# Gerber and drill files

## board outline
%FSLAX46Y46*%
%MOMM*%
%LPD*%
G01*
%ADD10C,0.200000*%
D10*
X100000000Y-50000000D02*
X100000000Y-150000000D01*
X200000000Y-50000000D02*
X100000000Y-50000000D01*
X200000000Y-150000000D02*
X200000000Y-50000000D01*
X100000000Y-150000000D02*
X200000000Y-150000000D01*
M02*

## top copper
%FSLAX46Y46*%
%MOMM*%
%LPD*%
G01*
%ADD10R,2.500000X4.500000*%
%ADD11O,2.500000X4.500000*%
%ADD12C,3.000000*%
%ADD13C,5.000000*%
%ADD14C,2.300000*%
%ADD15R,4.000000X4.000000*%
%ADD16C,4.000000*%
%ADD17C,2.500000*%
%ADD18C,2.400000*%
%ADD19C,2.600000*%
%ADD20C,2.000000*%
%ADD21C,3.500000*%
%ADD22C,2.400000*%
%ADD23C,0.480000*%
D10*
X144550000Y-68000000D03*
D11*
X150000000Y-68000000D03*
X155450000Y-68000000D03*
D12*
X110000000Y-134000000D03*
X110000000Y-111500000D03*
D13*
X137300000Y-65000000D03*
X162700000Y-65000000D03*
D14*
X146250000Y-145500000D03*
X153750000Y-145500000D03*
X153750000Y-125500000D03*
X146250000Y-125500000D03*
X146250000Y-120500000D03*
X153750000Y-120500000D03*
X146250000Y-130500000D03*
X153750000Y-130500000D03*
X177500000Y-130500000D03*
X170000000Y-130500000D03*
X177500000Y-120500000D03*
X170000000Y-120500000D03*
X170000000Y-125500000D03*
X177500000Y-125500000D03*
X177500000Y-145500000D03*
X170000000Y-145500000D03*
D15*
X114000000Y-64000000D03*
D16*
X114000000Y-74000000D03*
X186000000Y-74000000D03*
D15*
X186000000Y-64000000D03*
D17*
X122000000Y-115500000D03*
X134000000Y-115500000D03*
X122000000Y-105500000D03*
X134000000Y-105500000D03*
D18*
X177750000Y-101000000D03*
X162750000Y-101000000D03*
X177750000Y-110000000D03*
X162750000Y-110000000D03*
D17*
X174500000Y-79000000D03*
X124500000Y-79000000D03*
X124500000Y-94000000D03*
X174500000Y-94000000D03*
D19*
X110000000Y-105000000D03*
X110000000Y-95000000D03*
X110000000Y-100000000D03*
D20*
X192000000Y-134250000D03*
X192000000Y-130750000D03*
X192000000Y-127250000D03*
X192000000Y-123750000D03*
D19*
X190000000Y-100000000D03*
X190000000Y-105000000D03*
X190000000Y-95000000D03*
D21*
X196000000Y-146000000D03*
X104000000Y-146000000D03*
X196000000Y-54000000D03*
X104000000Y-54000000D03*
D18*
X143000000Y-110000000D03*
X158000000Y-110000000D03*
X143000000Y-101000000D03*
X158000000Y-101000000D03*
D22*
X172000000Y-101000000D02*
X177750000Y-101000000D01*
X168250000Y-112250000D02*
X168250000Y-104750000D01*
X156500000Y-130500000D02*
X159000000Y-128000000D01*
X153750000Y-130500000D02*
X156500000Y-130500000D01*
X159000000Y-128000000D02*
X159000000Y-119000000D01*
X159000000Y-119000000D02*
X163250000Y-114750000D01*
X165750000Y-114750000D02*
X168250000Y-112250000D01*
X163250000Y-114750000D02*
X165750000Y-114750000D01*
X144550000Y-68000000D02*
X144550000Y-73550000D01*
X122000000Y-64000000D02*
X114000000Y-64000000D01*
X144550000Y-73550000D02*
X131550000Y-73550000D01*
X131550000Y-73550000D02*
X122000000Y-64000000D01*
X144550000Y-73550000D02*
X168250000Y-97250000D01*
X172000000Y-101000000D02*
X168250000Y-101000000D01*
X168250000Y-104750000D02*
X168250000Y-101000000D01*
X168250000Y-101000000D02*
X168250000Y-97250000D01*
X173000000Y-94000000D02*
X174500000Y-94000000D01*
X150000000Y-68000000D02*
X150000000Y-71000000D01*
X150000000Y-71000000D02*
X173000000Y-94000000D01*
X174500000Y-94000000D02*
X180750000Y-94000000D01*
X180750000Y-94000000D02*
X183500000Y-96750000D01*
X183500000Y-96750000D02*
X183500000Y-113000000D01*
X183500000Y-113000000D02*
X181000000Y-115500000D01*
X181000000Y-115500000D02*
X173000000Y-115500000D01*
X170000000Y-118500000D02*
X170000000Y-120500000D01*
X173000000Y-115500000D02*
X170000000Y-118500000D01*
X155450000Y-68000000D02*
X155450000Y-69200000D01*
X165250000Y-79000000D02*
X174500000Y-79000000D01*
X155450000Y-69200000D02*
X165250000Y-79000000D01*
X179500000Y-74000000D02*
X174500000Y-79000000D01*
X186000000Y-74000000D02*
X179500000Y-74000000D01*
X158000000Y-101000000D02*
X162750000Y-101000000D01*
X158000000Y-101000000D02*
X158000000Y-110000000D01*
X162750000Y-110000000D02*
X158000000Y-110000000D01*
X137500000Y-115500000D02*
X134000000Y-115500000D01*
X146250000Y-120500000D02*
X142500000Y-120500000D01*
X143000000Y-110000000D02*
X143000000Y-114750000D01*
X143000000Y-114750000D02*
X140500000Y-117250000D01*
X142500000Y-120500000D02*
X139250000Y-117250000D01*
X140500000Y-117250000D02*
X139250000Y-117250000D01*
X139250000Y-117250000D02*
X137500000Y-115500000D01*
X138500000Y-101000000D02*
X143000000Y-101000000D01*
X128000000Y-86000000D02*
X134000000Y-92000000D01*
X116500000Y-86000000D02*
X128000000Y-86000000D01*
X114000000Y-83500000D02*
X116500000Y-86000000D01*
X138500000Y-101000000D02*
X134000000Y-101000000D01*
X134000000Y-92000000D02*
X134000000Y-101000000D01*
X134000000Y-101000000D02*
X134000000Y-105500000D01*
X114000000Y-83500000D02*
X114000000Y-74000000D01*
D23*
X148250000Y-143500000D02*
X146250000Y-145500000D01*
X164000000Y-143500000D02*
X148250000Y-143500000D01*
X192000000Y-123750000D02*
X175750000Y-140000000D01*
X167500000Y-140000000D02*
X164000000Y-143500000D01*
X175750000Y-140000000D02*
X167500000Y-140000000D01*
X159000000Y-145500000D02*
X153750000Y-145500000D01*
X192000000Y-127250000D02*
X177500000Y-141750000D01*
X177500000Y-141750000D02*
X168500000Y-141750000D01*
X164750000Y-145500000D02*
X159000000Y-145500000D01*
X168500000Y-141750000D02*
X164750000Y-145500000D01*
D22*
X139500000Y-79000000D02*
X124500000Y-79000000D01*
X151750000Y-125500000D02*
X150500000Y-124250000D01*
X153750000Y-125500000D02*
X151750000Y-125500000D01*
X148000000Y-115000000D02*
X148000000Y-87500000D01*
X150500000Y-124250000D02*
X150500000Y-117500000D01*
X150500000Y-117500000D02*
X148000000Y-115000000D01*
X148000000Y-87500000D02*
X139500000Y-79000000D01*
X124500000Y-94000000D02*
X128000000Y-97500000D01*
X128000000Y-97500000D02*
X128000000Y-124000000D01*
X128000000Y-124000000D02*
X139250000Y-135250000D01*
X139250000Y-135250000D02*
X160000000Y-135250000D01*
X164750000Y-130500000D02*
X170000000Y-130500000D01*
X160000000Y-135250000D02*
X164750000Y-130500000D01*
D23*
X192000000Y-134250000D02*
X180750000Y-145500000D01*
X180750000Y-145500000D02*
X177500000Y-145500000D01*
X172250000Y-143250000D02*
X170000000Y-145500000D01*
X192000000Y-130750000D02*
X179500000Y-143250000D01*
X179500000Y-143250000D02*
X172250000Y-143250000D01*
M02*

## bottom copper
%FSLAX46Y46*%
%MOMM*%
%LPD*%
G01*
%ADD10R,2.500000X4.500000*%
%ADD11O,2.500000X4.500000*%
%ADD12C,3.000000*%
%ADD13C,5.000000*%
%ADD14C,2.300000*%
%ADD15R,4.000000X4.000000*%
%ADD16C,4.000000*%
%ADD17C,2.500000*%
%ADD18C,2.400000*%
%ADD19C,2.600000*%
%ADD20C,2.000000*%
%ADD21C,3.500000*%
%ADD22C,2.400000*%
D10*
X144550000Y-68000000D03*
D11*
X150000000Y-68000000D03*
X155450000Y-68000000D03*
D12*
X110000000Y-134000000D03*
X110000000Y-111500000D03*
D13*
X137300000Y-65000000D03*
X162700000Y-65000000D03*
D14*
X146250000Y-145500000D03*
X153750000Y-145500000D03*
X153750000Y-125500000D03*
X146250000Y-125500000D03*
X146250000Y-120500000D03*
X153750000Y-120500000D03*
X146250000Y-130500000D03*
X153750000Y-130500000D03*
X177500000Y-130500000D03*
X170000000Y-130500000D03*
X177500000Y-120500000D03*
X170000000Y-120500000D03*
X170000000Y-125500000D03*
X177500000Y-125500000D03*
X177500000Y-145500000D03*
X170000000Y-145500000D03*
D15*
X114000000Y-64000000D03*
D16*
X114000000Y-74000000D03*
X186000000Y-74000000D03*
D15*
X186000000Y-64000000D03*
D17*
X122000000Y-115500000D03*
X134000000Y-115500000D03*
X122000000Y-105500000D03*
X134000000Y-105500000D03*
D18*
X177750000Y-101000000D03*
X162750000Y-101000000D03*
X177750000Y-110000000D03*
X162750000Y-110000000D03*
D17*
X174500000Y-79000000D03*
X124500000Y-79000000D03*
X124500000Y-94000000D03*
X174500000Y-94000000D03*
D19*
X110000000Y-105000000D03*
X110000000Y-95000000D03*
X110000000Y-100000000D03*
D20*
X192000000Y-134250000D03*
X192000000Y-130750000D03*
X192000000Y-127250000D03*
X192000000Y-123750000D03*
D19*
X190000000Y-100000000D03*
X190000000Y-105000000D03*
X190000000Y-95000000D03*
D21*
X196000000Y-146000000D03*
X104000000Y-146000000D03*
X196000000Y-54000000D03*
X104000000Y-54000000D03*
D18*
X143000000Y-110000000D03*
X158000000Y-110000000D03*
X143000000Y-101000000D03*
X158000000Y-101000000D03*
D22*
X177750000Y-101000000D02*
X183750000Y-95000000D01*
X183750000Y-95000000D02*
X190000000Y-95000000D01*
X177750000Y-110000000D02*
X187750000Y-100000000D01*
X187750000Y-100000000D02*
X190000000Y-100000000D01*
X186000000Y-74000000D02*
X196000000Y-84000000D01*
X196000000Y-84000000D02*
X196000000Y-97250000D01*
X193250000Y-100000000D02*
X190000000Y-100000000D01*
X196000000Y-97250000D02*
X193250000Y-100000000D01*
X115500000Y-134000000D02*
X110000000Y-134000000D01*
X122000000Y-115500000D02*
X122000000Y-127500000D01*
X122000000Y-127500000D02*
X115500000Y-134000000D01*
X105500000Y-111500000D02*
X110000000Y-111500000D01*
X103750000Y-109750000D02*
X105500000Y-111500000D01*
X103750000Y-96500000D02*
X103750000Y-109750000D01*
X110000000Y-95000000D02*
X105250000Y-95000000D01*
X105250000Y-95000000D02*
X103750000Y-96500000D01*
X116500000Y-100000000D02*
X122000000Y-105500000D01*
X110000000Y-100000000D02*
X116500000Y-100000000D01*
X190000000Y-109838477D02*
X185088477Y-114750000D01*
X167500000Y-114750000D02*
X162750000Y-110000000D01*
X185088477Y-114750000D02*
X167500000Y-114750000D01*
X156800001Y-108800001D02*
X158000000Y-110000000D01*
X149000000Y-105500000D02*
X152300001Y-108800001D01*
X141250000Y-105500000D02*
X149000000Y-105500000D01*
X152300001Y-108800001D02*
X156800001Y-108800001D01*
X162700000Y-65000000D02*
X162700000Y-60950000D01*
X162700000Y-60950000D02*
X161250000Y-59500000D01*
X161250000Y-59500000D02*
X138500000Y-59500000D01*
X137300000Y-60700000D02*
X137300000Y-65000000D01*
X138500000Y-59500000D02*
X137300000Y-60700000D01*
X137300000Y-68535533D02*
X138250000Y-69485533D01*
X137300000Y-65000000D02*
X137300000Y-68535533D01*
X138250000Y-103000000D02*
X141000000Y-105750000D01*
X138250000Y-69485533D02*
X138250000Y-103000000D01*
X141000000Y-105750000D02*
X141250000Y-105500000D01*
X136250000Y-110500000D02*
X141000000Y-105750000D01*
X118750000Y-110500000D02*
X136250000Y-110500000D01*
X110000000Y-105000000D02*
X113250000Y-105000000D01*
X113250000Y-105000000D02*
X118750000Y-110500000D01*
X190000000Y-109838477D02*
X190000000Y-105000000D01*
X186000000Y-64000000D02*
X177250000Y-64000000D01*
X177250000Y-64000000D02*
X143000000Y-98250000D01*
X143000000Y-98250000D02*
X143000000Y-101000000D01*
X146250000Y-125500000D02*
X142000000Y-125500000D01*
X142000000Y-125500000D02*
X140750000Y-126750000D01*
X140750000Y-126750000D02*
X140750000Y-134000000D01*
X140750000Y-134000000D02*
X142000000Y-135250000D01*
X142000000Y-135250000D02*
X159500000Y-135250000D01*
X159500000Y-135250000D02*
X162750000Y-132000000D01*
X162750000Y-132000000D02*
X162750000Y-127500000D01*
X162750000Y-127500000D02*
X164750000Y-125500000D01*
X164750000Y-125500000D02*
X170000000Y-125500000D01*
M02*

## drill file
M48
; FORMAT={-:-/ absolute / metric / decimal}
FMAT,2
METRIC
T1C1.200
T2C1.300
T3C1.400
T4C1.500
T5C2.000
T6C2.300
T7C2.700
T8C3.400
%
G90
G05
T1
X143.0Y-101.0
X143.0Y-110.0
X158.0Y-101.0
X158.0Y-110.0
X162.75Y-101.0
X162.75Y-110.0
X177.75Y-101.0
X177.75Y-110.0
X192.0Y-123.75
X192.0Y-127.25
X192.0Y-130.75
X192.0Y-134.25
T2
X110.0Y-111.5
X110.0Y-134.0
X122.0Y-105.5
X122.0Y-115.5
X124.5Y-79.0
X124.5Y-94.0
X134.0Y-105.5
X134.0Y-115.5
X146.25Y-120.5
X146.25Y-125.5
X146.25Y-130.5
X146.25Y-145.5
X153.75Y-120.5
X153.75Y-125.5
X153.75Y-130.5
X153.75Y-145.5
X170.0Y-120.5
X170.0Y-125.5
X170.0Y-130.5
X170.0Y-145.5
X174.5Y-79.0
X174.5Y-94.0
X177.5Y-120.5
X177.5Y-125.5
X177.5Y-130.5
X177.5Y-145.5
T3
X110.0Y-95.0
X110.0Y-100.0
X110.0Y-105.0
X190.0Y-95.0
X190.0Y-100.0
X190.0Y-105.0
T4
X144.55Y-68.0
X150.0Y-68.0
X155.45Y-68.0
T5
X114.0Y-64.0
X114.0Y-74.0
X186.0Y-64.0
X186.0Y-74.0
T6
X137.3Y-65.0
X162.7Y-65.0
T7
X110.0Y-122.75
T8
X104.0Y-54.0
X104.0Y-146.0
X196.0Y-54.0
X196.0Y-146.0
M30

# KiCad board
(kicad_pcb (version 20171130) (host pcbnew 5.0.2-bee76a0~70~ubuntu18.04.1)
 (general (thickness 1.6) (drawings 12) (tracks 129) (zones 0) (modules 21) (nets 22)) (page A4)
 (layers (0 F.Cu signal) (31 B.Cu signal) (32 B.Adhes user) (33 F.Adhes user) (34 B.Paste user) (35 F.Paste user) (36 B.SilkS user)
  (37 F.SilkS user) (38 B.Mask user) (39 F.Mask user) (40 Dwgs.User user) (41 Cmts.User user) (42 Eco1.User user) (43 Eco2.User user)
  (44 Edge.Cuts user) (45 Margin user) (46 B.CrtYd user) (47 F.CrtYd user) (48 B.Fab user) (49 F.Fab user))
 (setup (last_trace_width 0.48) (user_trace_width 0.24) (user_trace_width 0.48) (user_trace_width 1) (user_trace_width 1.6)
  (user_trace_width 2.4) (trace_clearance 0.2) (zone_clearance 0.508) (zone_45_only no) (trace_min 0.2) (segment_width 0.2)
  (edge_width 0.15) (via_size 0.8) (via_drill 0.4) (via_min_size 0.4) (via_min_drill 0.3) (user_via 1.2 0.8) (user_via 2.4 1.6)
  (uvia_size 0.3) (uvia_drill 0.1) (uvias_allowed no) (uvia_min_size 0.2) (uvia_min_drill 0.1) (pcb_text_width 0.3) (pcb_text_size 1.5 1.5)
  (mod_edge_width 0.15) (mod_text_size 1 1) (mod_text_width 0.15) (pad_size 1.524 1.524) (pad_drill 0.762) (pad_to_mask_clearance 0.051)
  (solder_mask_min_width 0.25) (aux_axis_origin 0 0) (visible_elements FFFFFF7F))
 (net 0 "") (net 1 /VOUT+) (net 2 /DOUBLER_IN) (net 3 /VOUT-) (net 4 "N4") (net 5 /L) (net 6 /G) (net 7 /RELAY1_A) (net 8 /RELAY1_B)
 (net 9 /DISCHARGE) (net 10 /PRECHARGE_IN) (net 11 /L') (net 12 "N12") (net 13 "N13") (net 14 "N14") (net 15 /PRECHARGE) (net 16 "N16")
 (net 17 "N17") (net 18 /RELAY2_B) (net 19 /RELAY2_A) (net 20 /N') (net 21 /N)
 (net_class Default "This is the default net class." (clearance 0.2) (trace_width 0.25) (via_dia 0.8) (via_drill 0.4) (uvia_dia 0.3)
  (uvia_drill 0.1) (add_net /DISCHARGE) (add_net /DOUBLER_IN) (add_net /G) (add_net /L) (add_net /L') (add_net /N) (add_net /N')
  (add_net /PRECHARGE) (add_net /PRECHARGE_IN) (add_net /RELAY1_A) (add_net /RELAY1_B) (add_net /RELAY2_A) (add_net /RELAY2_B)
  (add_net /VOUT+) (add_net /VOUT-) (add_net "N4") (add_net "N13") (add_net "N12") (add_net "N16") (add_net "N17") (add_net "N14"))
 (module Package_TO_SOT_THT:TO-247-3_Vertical (layer F.Cu) (at 144.55 68)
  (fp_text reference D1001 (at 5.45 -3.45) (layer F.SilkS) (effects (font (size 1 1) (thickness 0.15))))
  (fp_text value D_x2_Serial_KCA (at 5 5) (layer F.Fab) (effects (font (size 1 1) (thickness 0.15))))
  (pad 1 thru_hole rect (at 0 0) (size 2.5 4.5) (drill 1.5) (layers *.Cu *.Mask) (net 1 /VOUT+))
  (pad 2 thru_hole oval (at 5.45 0) (size 2.5 4.5) (drill 1.5) (layers *.Cu *.Mask) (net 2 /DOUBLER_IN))
  (pad 3 thru_hole oval (at 10.9 0) (size 2.5 4.5) (drill 1.5) (layers *.Cu *.Mask) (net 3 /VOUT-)))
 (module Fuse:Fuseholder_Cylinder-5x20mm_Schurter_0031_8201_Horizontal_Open (layer F.Cu) (at 110 134 90)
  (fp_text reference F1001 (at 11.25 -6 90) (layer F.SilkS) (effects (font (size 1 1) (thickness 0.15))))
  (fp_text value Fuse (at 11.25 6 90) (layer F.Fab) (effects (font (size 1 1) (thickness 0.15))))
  (pad 1 thru_hole circle (at 0 0 90) (size 3 3) (drill 1.3) (layers *.Cu *.Mask) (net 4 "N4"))
  (pad 2 thru_hole circle (at 22.5 0 90) (size 3 3) (drill 1.3) (layers *.Cu *.Mask) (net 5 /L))
  (pad "" np_thru_hole circle (at 11.25 0 90) (size 2.7 2.7) (drill 2.7) (layers *.Cu *.Mask)))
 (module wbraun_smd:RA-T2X (layer F.Cu) (at 150 68)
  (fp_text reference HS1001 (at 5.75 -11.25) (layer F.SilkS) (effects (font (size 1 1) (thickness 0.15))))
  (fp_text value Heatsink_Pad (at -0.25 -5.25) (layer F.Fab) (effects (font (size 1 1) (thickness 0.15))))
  (pad 1 thru_hole circle (at -12.7 -3) (size 5 5) (drill 2.3) (layers *.Cu *.Mask) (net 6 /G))
  (pad 1 thru_hole circle (at 12.7 -3) (size 5 5) (drill 2.3) (layers *.Cu *.Mask) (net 6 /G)))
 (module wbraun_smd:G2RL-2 (layer F.Cu) (at 150 133 90)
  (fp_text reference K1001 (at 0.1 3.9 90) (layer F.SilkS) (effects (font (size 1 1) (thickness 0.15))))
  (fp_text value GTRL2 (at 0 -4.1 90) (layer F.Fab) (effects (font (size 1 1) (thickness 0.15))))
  (pad 1 thru_hole circle (at -12.5 -3.75 90) (size 2.3 2.3) (drill 1.3) (layers *.Cu *.Mask) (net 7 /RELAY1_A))
  (pad 8 thru_hole circle (at -12.5 3.75 90) (size 2.3 2.3) (drill 1.3) (layers *.Cu *.Mask) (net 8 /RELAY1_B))
  (pad 6 thru_hole circle (at 7.5 3.75 90) (size 2.3 2.3) (drill 1.3) (layers *.Cu *.Mask) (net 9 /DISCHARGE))
  (pad 3 thru_hole circle (at 7.5 -3.75 90) (size 2.3 2.3) (drill 1.3) (layers *.Cu *.Mask) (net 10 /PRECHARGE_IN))
  (pad 4 thru_hole circle (at 12.5 -3.75 90) (size 2.3 2.3) (drill 1.3) (layers *.Cu *.Mask) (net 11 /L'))
  (pad 5 thru_hole circle (at 12.5 3.75 90) (size 2.3 2.3) (drill 1.3) (layers *.Cu *.Mask) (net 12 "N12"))
  (pad 2 thru_hole circle (at 2.5 -3.75 90) (size 2.3 2.3) (drill 1.3) (layers *.Cu *.Mask) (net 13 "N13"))
  (pad 7 thru_hole circle (at 2.5 3.75 90) (size 2.3 2.3) (drill 1.3) (layers *.Cu *.Mask) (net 1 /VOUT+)))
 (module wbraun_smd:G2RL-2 (layer F.Cu) (at 173.75 133 90)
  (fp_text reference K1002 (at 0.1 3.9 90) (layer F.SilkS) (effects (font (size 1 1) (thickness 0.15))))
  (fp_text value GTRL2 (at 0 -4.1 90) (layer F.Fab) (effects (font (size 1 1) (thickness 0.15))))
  (pad 7 thru_hole circle (at 2.5 3.75 90) (size 2.3 2.3) (drill 1.3) (layers *.Cu *.Mask) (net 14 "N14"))
  (pad 2 thru_hole circle (at 2.5 -3.75 90) (size 2.3 2.3) (drill 1.3) (layers *.Cu *.Mask) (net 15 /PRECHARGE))
  (pad 5 thru_hole circle (at 12.5 3.75 90) (size 2.3 2.3) (drill 1.3) (layers *.Cu *.Mask) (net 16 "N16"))
  (pad 4 thru_hole circle (at 12.5 -3.75 90) (size 2.3 2.3) (drill 1.3) (layers *.Cu *.Mask) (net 2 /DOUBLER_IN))
  (pad 3 thru_hole circle (at 7.5 -3.75 90) (size 2.3 2.3) (drill 1.3) (layers *.Cu *.Mask) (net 10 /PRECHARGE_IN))
  (pad 6 thru_hole circle (at 7.5 3.75 90) (size 2.3 2.3) (drill 1.3) (layers *.Cu *.Mask) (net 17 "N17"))
  (pad 8 thru_hole circle (at -12.5 3.75 90) (size 2.3 2.3) (drill 1.3) (layers *.Cu *.Mask) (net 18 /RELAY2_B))
  (pad 1 thru_hole circle (at -12.5 -3.75 90) (size 2.3 2.3) (drill 1.3) (layers *.Cu *.Mask) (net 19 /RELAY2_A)))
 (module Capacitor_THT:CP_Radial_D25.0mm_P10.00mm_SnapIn (layer F.Cu) (at 114 64 270)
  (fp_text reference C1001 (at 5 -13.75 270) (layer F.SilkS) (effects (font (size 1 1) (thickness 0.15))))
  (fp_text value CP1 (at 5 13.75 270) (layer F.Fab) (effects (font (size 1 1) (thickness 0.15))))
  (pad 1 thru_hole rect (at 0 0 270) (size 4 4) (drill 2) (layers *.Cu *.Mask) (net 1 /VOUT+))
  (pad 2 thru_hole circle (at 10 0 270) (size 4 4) (drill 2) (layers *.Cu *.Mask) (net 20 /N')))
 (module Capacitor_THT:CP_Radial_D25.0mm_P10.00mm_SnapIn (layer F.Cu) (at 186 64 270)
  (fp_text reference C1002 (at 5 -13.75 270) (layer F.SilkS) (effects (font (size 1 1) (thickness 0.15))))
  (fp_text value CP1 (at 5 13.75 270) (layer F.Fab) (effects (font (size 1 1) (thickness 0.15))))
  (pad 2 thru_hole circle (at 10 0 270) (size 4 4) (drill 2) (layers *.Cu *.Mask) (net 3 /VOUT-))
  (pad 1 thru_hole rect (at 0 0 270) (size 4 4) (drill 2) (layers *.Cu *.Mask) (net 20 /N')))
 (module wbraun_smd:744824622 (layer F.Cu) (at 128 110.5 90)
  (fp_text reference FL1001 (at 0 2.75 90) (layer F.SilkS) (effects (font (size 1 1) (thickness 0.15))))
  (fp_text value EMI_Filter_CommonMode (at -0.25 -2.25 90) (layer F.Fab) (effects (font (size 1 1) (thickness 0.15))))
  (pad 1 thru_hole circle (at -5 -6 90) (size 2.5 2.5) (drill 1.3) (layers *.Cu *.Mask) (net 4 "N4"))
  (pad 2 thru_hole circle (at -5 6 90) (size 2.5 2.5) (drill 1.3) (layers *.Cu *.Mask) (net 11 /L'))
  (pad 3 thru_hole circle (at 5 -6 90) (size 2.5 2.5) (drill 1.3) (layers *.Cu *.Mask) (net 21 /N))
  (pad 4 thru_hole circle (at 5 6 90) (size 2.5 2.5) (drill 1.3) (layers *.Cu *.Mask) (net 20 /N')))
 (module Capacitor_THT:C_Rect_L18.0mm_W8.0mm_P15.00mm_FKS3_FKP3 (layer F.Cu) (at 177.75 101 180)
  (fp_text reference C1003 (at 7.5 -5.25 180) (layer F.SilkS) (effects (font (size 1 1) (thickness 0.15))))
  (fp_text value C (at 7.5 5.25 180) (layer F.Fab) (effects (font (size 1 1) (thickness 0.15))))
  (pad 1 thru_hole circle (at 0 0 180) (size 2.4 2.4) (drill 1.2) (layers *.Cu *.Mask) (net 1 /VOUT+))
  (pad 2 thru_hole circle (at 15 0 180) (size 2.4 2.4) (drill 1.2) (layers *.Cu *.Mask) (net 6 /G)))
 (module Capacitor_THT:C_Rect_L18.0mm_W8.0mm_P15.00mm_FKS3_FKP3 (layer F.Cu) (at 162.75 110)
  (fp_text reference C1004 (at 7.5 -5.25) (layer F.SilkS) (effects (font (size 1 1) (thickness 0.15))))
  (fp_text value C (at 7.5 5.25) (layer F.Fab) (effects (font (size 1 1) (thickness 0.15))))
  (pad 2 thru_hole circle (at 15 0) (size 2.4 2.4) (drill 1.2) (layers *.Cu *.Mask) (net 3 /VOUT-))
  (pad 1 thru_hole circle (at 0 0) (size 2.4 2.4) (drill 1.2) (layers *.Cu *.Mask) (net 6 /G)))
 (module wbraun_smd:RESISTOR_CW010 (layer B.Cu) (at 149.5 79 180)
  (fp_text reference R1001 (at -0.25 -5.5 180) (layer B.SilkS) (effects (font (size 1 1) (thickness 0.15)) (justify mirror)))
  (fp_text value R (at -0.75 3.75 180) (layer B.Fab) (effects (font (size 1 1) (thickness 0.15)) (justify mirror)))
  (pad 1 thru_hole circle (at -25 0 180) (size 2.5 2.5) (drill 1.3) (layers *.Cu *.Mask) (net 3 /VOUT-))
  (pad 2 thru_hole circle (at 25 0 180) (size 2.5 2.5) (drill 1.3) (layers *.Cu *.Mask) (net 9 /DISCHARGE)))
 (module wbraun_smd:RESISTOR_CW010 (layer B.Cu) (at 149.5 94 180)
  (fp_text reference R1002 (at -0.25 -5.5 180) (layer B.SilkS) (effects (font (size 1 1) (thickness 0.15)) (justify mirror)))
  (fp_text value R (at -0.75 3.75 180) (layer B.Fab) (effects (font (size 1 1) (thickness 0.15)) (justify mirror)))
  (pad 2 thru_hole circle (at 25 0 180) (size 2.5 2.5) (drill 1.3) (layers *.Cu *.Mask) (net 15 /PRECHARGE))
  (pad 1 thru_hole circle (at -25 0 180) (size 2.5 2.5) (drill 1.3) (layers *.Cu *.Mask) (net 2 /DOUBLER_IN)))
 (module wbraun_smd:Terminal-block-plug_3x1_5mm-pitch (layer F.Cu) (at 110 100 90)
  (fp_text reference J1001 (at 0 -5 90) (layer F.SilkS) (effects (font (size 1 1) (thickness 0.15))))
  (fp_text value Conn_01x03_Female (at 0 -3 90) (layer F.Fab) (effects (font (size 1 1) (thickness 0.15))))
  (pad 1 thru_hole circle (at -5 0 90) (size 2.6 2.6) (drill 1.4) (layers *.Cu *.Mask) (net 6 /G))
  (pad 3 thru_hole circle (at 5 0 90) (size 2.6 2.6) (drill 1.4) (layers *.Cu *.Mask) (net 5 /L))
  (pad 2 thru_hole circle (at 0 0 90) (size 2.6 2.6) (drill 1.4) (layers *.Cu *.Mask) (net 21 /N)))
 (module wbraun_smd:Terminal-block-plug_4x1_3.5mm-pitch (layer F.Cu) (at 192 129 270)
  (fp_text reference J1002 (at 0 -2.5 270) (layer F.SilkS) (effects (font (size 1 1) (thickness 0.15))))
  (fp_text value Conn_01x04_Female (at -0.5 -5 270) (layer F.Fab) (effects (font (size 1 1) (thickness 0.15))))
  (pad 4 thru_hole circle (at 5.25 0 270) (size 2 2) (drill 1.2) (layers *.Cu *.Mask) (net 18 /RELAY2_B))
  (pad 3 thru_hole circle (at 1.75 0 270) (size 2 2) (drill 1.2) (layers *.Cu *.Mask) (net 19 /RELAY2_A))
  (pad 2 thru_hole circle (at -1.75 0 270) (size 2 2) (drill 1.2) (layers *.Cu *.Mask) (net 8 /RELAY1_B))
  (pad 1 thru_hole circle (at -5.25 0 270) (size 2 2) (drill 1.2) (layers *.Cu *.Mask) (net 7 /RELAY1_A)))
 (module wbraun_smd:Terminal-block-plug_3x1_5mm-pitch (layer F.Cu) (at 190 100 270)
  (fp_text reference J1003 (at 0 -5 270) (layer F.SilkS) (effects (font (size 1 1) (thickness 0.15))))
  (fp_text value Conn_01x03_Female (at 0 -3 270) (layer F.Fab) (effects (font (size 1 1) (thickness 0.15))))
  (pad 2 thru_hole circle (at 0 0 270) (size 2.6 2.6) (drill 1.4) (layers *.Cu *.Mask) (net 3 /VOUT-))
  (pad 3 thru_hole circle (at 5 0 270) (size 2.6 2.6) (drill 1.4) (layers *.Cu *.Mask) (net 6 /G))
  (pad 1 thru_hole circle (at -5 0 270) (size 2.6 2.6) (drill 1.4) (layers *.Cu *.Mask) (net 1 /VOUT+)))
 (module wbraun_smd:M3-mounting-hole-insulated (layer F.Cu) (at 196 146)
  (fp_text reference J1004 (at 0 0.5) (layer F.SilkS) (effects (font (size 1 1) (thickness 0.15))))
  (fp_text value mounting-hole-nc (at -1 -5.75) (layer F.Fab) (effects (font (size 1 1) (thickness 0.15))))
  (pad "" np_thru_hole circle (at 0 0) (size 3.5 3.5) (drill 3.4) (layers *.Cu *.Mask)))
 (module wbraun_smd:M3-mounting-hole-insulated (layer F.Cu) (at 104 146)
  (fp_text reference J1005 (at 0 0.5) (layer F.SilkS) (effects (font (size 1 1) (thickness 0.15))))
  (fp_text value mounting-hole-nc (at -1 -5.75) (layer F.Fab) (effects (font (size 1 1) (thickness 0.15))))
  (pad "" np_thru_hole circle (at 0 0) (size 3.5 3.5) (drill 3.4) (layers *.Cu *.Mask)))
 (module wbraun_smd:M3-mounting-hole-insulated (layer F.Cu) (at 196 54)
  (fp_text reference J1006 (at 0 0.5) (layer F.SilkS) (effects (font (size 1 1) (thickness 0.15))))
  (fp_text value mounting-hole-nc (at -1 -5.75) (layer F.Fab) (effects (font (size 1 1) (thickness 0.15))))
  (pad "" np_thru_hole circle (at 0 0) (size 3.5 3.5) (drill 3.4) (layers *.Cu *.Mask)))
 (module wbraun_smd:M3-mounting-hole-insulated (layer F.Cu) (at 104 54)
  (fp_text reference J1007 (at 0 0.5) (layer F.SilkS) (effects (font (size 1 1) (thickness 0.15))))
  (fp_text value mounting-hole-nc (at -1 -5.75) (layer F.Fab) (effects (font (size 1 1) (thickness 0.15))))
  (pad "" np_thru_hole circle (at 0 0) (size 3.5 3.5) (drill 3.4) (layers *.Cu *.Mask)))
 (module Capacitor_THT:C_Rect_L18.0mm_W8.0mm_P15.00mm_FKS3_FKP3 (layer F.Cu) (at 143 110)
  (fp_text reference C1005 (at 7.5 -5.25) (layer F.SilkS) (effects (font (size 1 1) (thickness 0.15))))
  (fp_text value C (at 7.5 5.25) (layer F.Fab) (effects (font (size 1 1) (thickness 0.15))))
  (pad 1 thru_hole circle (at 0 0) (size 2.4 2.4) (drill 1.2) (layers *.Cu *.Mask) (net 11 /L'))
  (pad 2 thru_hole circle (at 15 0) (size 2.4 2.4) (drill 1.2) (layers *.Cu *.Mask) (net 6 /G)))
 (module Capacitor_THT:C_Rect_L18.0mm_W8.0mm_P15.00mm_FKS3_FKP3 (layer F.Cu) (at 158 101 180)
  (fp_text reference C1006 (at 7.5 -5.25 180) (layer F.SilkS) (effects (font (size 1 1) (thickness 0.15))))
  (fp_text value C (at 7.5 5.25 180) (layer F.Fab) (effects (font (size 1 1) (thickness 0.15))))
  (pad 2 thru_hole circle (at 15 0 180) (size 2.4 2.4) (drill 1.2) (layers *.Cu *.Mask) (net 20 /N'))
  (pad 1 thru_hole circle (at 0 0 180) (size 2.4 2.4) (drill 1.2) (layers *.Cu *.Mask) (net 6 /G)))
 (gr_line (start 100 50) (end 100 150) (layer Edge.Cuts) (width 0.2))
 (gr_line (start 200 50) (end 100 50) (layer Edge.Cuts) (width 0.2))
 (gr_line (start 200 150) (end 200 50) (layer Edge.Cuts) (width 0.2))
 (gr_line (start 100 150) (end 200 150) (layer Edge.Cuts) (width 0.2))
 (segment (start 172 101) (end 177.75 101) (width 2.4) (layer F.Cu) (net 1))
 (segment (start 168.25 112.25) (end 168.25 104.75) (width 2.4) (layer F.Cu) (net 1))
 (segment (start 156.5 130.5) (end 159 128) (width 2.4) (layer F.Cu) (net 1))
 (segment (start 153.75 130.5) (end 156.5 130.5) (width 2.4) (layer F.Cu) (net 1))
 (segment (start 159 128) (end 159 119) (width 2.4) (layer F.Cu) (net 1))
 (segment (start 159 119) (end 163.25 114.75) (width 2.4) (layer F.Cu) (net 1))
 (segment (start 165.75 114.75) (end 168.25 112.25) (width 2.4) (layer F.Cu) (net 1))
 (segment (start 163.25 114.75) (end 165.75 114.75) (width 2.4) (layer F.Cu) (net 1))
 (segment (start 144.55 68) (end 144.55 73.55) (width 2.4) (layer F.Cu) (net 1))
 (segment (start 122 64) (end 114 64) (width 2.4) (layer F.Cu) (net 1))
 (segment (start 144.55 73.55) (end 131.55 73.55) (width 2.4) (layer F.Cu) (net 1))
 (segment (start 131.55 73.55) (end 122 64) (width 2.4) (layer F.Cu) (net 1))
 (segment (start 177.75 101) (end 183.75 95) (width 2.4) (layer B.Cu) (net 1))
 (segment (start 183.75 95) (end 190 95) (width 2.4) (layer B.Cu) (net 1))
 (segment (start 144.55 73.55) (end 168.25 97.25) (width 2.4) (layer F.Cu) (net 1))
 (segment (start 172 101) (end 168.25 101) (width 2.4) (layer F.Cu) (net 1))
 (segment (start 168.25 104.75) (end 168.25 101) (width 2.4) (layer F.Cu) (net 1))
 (segment (start 168.25 101) (end 168.25 97.25) (width 2.4) (layer F.Cu) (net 1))
 (segment (start 173 94) (end 174.5 94) (width 2.4) (layer F.Cu) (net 2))
 (segment (start 150 68) (end 150 71) (width 2.4) (layer F.Cu) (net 2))
 (segment (start 150 71) (end 173 94) (width 2.4) (layer F.Cu) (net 2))
 (segment (start 174.5 94) (end 180.75 94) (width 2.4) (layer F.Cu) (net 2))
 (segment (start 180.75 94) (end 183.5 96.75) (width 2.4) (layer F.Cu) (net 2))
 (segment (start 183.5 96.75) (end 183.5 113) (width 2.4) (layer F.Cu) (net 2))
 (segment (start 183.5 113) (end 181 115.5) (width 2.4) (layer F.Cu) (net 2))
 (segment (start 181 115.5) (end 173 115.5) (width 2.4) (layer F.Cu) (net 2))
 (segment (start 170 118.5) (end 170 120.5) (width 2.4) (layer F.Cu) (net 2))
 (segment (start 173 115.5) (end 170 118.5) (width 2.4) (layer F.Cu) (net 2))
 (segment (start 155.45 68) (end 155.45 69.2) (width 2.4) (layer F.Cu) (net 3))
 (segment (start 165.25 79) (end 174.5 79) (width 2.4) (layer F.Cu) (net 3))
 (segment (start 155.45 69.2) (end 165.25 79) (width 2.4) (layer F.Cu) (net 3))
 (segment (start 179.5 74) (end 174.5 79) (width 2.4) (layer F.Cu) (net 3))
 (segment (start 186 74) (end 179.5 74) (width 2.4) (layer F.Cu) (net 3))
 (segment (start 177.75 110) (end 187.75 100) (width 2.4) (layer B.Cu) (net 3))
 (segment (start 187.75 100) (end 190 100) (width 2.4) (layer B.Cu) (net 3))
 (segment (start 186 74) (end 196 84) (width 2.4) (layer B.Cu) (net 3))
 (segment (start 196 84) (end 196 97.25) (width 2.4) (layer B.Cu) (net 3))
 (segment (start 193.25 100) (end 190 100) (width 2.4) (layer B.Cu) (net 3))
 (segment (start 196 97.25) (end 193.25 100) (width 2.4) (layer B.Cu) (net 3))
 (segment (start 115.5 134) (end 110 134) (width 2.4) (layer B.Cu) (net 4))
 (segment (start 122 115.5) (end 122 127.5) (width 2.4) (layer B.Cu) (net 4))
 (segment (start 122 127.5) (end 115.5 134) (width 2.4) (layer B.Cu) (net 4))
 (segment (start 105.5 111.5) (end 110 111.5) (width 2.4) (layer B.Cu) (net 5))
 (segment (start 103.75 109.75) (end 105.5 111.5) (width 2.4) (layer B.Cu) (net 5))
 (segment (start 103.75 96.5) (end 103.75 109.75) (width 2.4) (layer B.Cu) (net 5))
 (segment (start 110 95) (end 105.25 95) (width 2.4) (layer B.Cu) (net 5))
 (segment (start 105.25 95) (end 103.75 96.5) (width 2.4) (layer B.Cu) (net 5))
 (segment (start 116.5 100) (end 122 105.5) (width 2.4) (layer B.Cu) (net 21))
 (segment (start 110 100) (end 116.5 100) (width 2.4) (layer B.Cu) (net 21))
 (segment (start 158 101) (end 162.75 101) (width 2.4) (layer F.Cu) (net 6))
 (segment (start 158 101) (end 158 110) (width 2.4) (layer F.Cu) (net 6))
 (segment (start 162.75 110) (end 158 110) (width 2.4) (layer F.Cu) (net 6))
 (segment (start 190 109.838477) (end 185.088477 114.75) (width 2.4) (layer B.Cu) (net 6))
 (segment (start 167.5 114.75) (end 162.75 110) (width 2.4) (layer B.Cu) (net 6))
 (segment (start 185.088477 114.75) (end 167.5 114.75) (width 2.4) (layer B.Cu) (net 6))
 (segment (start 156.800001 108.800001) (end 158 110) (width 2.4) (layer B.Cu) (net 6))
 (segment (start 149 105.5) (end 152.300001 108.800001) (width 2.4) (layer B.Cu) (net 6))
 (segment (start 141.25 105.5) (end 149 105.5) (width 2.4) (layer B.Cu) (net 6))
 (segment (start 152.300001 108.800001) (end 156.800001 108.800001) (width 2.4) (layer B.Cu) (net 6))
 (segment (start 162.7 65) (end 162.7 60.95) (width 2.4) (layer B.Cu) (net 6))
 (segment (start 162.7 60.95) (end 161.25 59.5) (width 2.4) (layer B.Cu) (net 6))
 (segment (start 161.25 59.5) (end 138.5 59.5) (width 2.4) (layer B.Cu) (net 6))
 (segment (start 137.3 60.7) (end 137.3 65) (width 2.4) (layer B.Cu) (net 6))
 (segment (start 138.5 59.5) (end 137.3 60.7) (width 2.4) (layer B.Cu) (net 6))
 (segment (start 137.3 68.535533) (end 138.25 69.485533) (width 2.4) (layer B.Cu) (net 6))
 (segment (start 137.3 65) (end 137.3 68.535533) (width 2.4) (layer B.Cu) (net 6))
 (segment (start 138.25 103) (end 141 105.75) (width 2.4) (layer B.Cu) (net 6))
 (segment (start 138.25 69.485533) (end 138.25 103) (width 2.4) (layer B.Cu) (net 6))
 (segment (start 141 105.75) (end 141.25 105.5) (width 2.4) (layer B.Cu) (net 6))
 (segment (start 136.25 110.5) (end 141 105.75) (width 2.4) (layer B.Cu) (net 6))
 (segment (start 118.75 110.5) (end 136.25 110.5) (width 2.4) (layer B.Cu) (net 6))
 (segment (start 110 105) (end 113.25 105) (width 2.4) (layer B.Cu) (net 6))
 (segment (start 113.25 105) (end 118.75 110.5) (width 2.4) (layer B.Cu) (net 6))
 (segment (start 190 109.838477) (end 190 105) (width 2.4) (layer B.Cu) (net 6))
 (segment (start 137.5 115.5) (end 134 115.5) (width 2.4) (layer F.Cu) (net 11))
 (segment (start 146.25 120.5) (end 142.5 120.5) (width 2.4) (layer F.Cu) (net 11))
 (segment (start 143 110) (end 143 114.75) (width 2.4) (layer F.Cu) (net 11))
 (segment (start 143 114.75) (end 140.5 117.25) (width 2.4) (layer F.Cu) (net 11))
 (segment (start 142.5 120.5) (end 139.25 117.25) (width 2.4) (layer F.Cu) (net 11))
 (segment (start 140.5 117.25) (end 139.25 117.25) (width 2.4) (layer F.Cu) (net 11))
 (segment (start 139.25 117.25) (end 137.5 115.5) (width 2.4) (layer F.Cu) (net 11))
 (segment (start 138.5 101) (end 143 101) (width 2.4) (layer F.Cu) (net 20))
 (segment (start 128 86) (end 134 92) (width 2.4) (layer F.Cu) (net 20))
 (segment (start 116.5 86) (end 128 86) (width 2.4) (layer F.Cu) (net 20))
 (segment (start 114 83.5) (end 116.5 86) (width 2.4) (layer F.Cu) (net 20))
 (segment (start 186 64) (end 177.25 64) (width 2.4) (layer B.Cu) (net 20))
 (segment (start 177.25 64) (end 143 98.25) (width 2.4) (layer B.Cu) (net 20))
 (segment (start 143 98.25) (end 143 101) (width 2.4) (layer B.Cu) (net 20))
 (segment (start 138.5 101) (end 134 101) (width 2.4) (layer F.Cu) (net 20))
 (segment (start 134 92) (end 134 101) (width 2.4) (layer F.Cu) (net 20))
 (segment (start 134 101) (end 134 105.5) (width 2.4) (layer F.Cu) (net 20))
 (segment (start 114 83.5) (end 114 74) (width 2.4) (layer F.Cu) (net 20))
 (segment (start 148.25 143.5) (end 146.25 145.5) (width 0.48) (layer F.Cu) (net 7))
 (segment (start 164 143.5) (end 148.25 143.5) (width 0.48) (layer F.Cu) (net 7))
 (segment (start 192 123.75) (end 175.75 140) (width 0.48) (layer F.Cu) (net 7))
 (segment (start 167.5 140) (end 164 143.5) (width 0.48) (layer F.Cu) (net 7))
 (segment (start 175.75 140) (end 167.5 140) (width 0.48) (layer F.Cu) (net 7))
 (segment (start 159 145.5) (end 153.75 145.5) (width 0.48) (layer F.Cu) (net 8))
 (segment (start 192 127.25) (end 177.5 141.75) (width 0.48) (layer F.Cu) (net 8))
 (segment (start 177.5 141.75) (end 168.5 141.75) (width 0.48) (layer F.Cu) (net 8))
 (segment (start 164.75 145.5) (end 159 145.5) (width 0.48) (layer F.Cu) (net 8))
 (segment (start 168.5 141.75) (end 164.75 145.5) (width 0.48) (layer F.Cu) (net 8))
 (segment (start 146.25 125.5) (end 142 125.5) (width 2.4) (layer B.Cu) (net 10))
 (segment (start 142 125.5) (end 140.75 126.75) (width 2.4) (layer B.Cu) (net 10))
 (segment (start 140.75 126.75) (end 140.75 134) (width 2.4) (layer B.Cu) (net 10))
 (segment (start 140.75 134) (end 142 135.25) (width 2.4) (layer B.Cu) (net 10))
 (segment (start 142 135.25) (end 159.5 135.25) (width 2.4) (layer B.Cu) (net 10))
 (segment (start 159.5 135.25) (end 162.75 132) (width 2.4) (layer B.Cu) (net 10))
 (segment (start 162.75 132) (end 162.75 127.5) (width 2.4) (layer B.Cu) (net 10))
 (segment (start 162.75 127.5) (end 164.75 125.5) (width 2.4) (layer B.Cu) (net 10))
 (segment (start 164.75 125.5) (end 170 125.5) (width 2.4) (layer B.Cu) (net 10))
 (segment (start 139.5 79) (end 124.5 79) (width 2.4) (layer F.Cu) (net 9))
 (segment (start 151.75 125.5) (end 150.5 124.25) (width 2.4) (layer F.Cu) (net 9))
 (segment (start 153.75 125.5) (end 151.75 125.5) (width 2.4) (layer F.Cu) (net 9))
 (segment (start 148 115) (end 148 87.5) (width 2.4) (layer F.Cu) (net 9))
 (segment (start 150.5 124.25) (end 150.5 117.5) (width 2.4) (layer F.Cu) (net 9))
 (segment (start 150.5 117.5) (end 148 115) (width 2.4) (layer F.Cu) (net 9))
 (segment (start 148 87.5) (end 139.5 79) (width 2.4) (layer F.Cu) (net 9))
 (segment (start 124.5 94) (end 128 97.5) (width 2.4) (layer F.Cu) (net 15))
 (segment (start 128 97.5) (end 128 124) (width 2.4) (layer F.Cu) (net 15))
 (segment (start 128 124) (end 139.25 135.25) (width 2.4) (layer F.Cu) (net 15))
 (segment (start 139.25 135.25) (end 160 135.25) (width 2.4) (layer F.Cu) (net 15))
 (segment (start 164.75 130.5) (end 170 130.5) (width 2.4) (layer F.Cu) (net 15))
 (segment (start 160 135.25) (end 164.75 130.5) (width 2.4) (layer F.Cu) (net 15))
 (segment (start 192 134.25) (end 180.75 145.5) (width 0.48) (layer F.Cu) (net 18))
 (segment (start 180.75 145.5) (end 177.5 145.5) (width 0.48) (layer F.Cu) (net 18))
 (segment (start 172.25 143.25) (end 170 145.5) (width 0.48) (layer F.Cu) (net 19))
 (segment (start 192 130.75) (end 179.5 143.25) (width 0.48) (layer F.Cu) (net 19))
 (segment (start 179.5 143.25) (end 172.25 143.25) (width 0.48) (layer F.Cu) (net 19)))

